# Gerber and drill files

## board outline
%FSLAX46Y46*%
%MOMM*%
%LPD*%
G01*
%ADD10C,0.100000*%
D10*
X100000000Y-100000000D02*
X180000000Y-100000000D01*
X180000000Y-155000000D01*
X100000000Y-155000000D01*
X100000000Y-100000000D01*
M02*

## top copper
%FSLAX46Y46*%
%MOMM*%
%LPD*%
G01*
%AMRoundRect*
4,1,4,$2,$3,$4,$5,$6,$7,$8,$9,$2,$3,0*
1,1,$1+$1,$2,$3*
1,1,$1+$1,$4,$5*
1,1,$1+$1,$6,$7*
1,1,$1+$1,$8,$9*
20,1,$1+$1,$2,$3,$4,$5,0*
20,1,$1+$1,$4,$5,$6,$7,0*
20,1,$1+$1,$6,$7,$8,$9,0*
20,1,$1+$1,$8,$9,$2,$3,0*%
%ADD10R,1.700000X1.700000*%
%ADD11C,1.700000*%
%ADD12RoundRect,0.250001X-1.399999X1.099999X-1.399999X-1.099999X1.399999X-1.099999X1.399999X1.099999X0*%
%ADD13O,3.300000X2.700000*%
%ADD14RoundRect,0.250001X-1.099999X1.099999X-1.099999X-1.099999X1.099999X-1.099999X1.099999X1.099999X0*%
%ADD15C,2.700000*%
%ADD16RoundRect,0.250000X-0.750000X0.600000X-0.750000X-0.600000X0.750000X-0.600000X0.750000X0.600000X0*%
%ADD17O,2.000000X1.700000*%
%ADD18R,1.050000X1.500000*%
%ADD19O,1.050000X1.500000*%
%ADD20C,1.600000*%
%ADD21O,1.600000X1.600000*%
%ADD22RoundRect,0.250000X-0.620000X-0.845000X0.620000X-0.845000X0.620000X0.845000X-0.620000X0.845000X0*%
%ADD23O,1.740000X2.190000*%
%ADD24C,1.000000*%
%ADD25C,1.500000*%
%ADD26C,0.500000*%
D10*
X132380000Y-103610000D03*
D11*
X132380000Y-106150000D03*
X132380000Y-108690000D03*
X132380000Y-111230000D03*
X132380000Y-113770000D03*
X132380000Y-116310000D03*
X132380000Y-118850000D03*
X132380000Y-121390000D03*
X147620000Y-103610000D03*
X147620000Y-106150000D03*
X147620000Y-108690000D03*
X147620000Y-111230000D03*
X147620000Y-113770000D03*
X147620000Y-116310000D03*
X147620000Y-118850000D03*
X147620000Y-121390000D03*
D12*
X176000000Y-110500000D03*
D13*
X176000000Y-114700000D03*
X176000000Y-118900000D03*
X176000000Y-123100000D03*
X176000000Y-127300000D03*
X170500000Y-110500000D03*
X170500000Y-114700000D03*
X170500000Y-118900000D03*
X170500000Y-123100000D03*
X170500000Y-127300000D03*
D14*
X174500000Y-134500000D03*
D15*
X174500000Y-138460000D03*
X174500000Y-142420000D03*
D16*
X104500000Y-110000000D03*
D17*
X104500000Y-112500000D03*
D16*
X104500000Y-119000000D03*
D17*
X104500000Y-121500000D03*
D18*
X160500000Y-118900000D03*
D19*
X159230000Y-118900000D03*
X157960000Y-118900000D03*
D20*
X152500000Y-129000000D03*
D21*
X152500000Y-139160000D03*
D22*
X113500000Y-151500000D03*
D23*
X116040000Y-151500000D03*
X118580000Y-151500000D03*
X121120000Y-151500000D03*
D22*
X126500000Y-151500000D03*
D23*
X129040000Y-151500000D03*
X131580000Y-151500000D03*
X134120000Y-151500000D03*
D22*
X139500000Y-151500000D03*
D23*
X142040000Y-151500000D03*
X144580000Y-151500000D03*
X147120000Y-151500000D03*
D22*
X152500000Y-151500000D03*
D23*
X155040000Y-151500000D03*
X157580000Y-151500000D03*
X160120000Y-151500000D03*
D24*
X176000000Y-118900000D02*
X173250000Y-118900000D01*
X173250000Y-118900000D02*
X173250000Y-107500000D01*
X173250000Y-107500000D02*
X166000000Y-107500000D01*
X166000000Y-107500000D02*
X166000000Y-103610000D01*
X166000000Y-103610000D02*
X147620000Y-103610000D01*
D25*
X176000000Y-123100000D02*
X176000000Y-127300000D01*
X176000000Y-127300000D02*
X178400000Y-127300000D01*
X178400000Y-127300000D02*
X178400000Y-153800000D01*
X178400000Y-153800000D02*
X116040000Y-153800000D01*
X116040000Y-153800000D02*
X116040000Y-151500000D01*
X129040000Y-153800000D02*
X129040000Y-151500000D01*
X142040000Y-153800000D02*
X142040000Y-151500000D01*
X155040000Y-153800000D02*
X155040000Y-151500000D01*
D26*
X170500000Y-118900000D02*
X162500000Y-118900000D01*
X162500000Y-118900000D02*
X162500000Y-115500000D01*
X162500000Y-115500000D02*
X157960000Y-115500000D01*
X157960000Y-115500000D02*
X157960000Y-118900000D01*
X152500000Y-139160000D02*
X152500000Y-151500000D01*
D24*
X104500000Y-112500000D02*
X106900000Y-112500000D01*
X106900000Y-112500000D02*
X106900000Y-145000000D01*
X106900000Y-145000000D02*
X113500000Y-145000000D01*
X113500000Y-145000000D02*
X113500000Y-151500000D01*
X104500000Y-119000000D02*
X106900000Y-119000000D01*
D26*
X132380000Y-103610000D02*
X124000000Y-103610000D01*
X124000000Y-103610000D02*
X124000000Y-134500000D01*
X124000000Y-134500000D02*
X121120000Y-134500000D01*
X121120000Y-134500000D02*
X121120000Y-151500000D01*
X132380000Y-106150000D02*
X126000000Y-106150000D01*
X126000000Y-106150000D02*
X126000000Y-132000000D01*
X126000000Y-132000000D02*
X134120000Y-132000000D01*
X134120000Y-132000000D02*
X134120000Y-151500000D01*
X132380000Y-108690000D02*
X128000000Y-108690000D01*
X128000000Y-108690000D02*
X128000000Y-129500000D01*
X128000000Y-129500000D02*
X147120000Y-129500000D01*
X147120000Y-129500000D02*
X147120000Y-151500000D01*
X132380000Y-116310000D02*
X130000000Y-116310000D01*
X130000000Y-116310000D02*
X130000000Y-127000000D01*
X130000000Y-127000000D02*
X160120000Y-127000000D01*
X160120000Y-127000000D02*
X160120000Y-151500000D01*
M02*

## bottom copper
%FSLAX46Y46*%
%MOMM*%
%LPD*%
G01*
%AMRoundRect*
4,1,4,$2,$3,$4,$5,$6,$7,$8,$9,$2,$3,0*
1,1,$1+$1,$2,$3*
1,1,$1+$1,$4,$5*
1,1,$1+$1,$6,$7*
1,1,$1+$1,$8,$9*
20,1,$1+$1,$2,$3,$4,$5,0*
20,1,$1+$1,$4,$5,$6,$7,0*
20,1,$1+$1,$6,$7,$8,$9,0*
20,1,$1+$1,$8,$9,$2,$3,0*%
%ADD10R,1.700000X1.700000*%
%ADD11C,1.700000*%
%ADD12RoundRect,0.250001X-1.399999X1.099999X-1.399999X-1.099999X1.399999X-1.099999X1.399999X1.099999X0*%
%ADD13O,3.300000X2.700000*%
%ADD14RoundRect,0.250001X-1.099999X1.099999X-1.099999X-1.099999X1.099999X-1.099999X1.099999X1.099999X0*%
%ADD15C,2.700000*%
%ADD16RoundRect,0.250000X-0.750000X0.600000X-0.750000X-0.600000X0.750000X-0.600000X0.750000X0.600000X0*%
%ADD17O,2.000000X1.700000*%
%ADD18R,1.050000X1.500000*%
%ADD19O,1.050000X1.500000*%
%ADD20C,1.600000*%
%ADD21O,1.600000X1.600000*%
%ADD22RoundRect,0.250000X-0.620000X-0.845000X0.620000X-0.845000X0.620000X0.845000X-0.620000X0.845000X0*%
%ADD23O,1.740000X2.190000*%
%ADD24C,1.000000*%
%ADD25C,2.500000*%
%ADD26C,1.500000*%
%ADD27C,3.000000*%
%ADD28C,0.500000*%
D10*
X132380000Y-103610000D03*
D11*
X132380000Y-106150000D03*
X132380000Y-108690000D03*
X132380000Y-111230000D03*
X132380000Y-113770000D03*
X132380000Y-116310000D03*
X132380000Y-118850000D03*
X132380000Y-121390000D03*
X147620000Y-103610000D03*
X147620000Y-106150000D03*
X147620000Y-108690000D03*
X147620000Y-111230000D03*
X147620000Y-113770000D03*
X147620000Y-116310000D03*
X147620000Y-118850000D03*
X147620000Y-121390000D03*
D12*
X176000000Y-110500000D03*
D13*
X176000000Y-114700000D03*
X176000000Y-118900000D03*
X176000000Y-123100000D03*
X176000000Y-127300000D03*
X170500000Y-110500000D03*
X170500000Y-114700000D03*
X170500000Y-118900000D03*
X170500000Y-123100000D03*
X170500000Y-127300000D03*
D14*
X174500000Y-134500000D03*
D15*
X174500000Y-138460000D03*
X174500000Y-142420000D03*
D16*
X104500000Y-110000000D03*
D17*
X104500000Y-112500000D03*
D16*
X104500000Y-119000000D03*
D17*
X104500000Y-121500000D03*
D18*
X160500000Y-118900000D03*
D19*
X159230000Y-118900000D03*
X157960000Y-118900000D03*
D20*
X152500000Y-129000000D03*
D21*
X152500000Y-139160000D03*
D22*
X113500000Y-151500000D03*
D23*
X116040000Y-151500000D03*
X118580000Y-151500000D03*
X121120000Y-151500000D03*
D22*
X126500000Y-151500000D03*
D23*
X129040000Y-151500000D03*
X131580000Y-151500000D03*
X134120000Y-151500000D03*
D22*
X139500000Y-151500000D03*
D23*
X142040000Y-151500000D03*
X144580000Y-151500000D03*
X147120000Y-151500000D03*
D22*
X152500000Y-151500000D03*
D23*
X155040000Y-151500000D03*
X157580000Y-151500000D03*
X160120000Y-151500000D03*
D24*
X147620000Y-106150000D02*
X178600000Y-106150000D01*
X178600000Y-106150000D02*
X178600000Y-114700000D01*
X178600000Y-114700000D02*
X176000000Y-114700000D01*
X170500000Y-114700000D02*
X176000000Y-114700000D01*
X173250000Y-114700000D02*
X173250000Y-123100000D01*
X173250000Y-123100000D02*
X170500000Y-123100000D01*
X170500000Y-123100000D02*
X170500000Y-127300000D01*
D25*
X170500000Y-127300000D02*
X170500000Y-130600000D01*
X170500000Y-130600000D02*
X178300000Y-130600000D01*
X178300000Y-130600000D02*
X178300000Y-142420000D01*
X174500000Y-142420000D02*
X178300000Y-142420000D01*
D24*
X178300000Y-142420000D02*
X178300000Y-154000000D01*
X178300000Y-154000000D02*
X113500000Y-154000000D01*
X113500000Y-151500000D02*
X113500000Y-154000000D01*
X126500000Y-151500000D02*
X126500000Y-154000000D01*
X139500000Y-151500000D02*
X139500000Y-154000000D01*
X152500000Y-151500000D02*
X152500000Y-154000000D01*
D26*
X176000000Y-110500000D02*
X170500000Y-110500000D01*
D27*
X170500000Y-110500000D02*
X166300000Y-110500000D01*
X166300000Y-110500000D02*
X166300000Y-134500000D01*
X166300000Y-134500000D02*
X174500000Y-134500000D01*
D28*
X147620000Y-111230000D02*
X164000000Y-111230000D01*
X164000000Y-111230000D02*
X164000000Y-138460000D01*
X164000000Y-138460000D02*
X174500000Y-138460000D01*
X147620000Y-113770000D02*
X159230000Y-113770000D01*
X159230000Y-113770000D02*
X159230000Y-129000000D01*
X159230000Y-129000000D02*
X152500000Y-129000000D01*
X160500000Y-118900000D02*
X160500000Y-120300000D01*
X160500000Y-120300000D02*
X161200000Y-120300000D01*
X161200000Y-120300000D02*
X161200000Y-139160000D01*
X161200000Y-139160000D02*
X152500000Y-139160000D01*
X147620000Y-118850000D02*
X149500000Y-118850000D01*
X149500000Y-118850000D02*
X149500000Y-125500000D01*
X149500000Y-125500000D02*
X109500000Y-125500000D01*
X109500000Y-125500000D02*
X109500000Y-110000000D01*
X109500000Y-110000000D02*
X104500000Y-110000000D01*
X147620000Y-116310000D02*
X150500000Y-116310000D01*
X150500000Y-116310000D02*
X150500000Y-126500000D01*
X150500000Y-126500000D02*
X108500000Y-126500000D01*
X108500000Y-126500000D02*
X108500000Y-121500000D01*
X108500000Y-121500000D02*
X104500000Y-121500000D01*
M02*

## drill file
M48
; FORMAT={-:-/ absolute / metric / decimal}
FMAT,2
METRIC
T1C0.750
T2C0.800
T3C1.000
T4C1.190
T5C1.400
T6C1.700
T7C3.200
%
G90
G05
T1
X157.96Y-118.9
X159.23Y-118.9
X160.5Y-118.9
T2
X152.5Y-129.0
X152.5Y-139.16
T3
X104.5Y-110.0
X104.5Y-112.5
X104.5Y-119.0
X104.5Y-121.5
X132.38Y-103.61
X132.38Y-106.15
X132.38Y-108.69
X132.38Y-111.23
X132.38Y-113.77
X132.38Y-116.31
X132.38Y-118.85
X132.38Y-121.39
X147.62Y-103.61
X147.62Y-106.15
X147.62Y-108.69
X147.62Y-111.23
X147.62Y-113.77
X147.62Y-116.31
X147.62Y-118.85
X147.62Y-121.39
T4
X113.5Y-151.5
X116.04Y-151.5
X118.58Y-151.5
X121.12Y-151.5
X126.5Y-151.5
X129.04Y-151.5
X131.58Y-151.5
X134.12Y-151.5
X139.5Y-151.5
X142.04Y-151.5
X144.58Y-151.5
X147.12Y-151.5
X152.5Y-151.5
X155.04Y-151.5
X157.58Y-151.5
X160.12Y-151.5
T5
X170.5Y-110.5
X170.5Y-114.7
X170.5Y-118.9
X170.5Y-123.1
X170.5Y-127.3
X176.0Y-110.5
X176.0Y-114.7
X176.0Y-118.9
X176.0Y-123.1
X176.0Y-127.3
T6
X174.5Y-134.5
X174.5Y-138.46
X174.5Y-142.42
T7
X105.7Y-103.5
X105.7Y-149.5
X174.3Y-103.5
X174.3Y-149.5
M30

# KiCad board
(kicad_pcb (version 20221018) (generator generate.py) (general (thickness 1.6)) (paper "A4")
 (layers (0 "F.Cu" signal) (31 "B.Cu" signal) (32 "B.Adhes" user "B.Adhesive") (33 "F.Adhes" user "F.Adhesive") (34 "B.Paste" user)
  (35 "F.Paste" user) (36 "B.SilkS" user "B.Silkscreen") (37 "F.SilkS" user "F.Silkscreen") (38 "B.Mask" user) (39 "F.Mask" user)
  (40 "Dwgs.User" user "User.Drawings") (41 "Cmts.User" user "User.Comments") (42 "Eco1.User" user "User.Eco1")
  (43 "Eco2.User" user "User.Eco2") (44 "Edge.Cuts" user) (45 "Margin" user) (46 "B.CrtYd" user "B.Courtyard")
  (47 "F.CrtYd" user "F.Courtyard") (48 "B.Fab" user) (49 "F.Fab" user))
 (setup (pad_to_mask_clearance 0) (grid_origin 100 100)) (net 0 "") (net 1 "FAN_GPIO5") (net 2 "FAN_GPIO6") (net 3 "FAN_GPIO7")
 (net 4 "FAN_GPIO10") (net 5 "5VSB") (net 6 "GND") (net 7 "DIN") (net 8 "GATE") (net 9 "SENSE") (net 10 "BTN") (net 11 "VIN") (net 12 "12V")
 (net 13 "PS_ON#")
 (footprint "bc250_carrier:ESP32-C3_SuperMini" (layer "F.Cu") (at 140 112.5 0)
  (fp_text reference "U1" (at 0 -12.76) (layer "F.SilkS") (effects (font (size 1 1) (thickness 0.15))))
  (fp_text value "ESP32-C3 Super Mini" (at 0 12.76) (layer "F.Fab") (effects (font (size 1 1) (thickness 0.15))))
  (pad "1" thru_hole rect (at -7.62 -8.89) (size 1.7 1.7) (drill 1) (layers "*.Cu" "*.Mask") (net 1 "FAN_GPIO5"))
  (pad "2" thru_hole circle (at -7.62 -6.35) (size 1.7 1.7) (drill 1) (layers "*.Cu" "*.Mask") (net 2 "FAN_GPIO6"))
  (pad "3" thru_hole circle (at -7.62 -3.81) (size 1.7 1.7) (drill 1) (layers "*.Cu" "*.Mask") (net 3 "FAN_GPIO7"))
  (pad "4" thru_hole circle (at -7.62 -1.27) (size 1.7 1.7) (drill 1) (layers "*.Cu" "*.Mask"))
  (pad "5" thru_hole circle (at -7.62 1.27) (size 1.7 1.7) (drill 1) (layers "*.Cu" "*.Mask"))
  (pad "6" thru_hole circle (at -7.62 3.81) (size 1.7 1.7) (drill 1) (layers "*.Cu" "*.Mask") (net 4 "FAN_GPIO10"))
  (pad "7" thru_hole circle (at -7.62 6.35) (size 1.7 1.7) (drill 1) (layers "*.Cu" "*.Mask"))
  (pad "8" thru_hole circle (at -7.62 8.89) (size 1.7 1.7) (drill 1) (layers "*.Cu" "*.Mask"))
  (pad "9" thru_hole circle (at 7.62 -8.89) (size 1.7 1.7) (drill 1) (layers "*.Cu" "*.Mask") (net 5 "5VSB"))
  (pad "10" thru_hole circle (at 7.62 -6.35) (size 1.7 1.7) (drill 1) (layers "*.Cu" "*.Mask") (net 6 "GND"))
  (pad "11" thru_hole circle (at 7.62 -3.81) (size 1.7 1.7) (drill 1) (layers "*.Cu" "*.Mask"))
  (pad "12" thru_hole circle (at 7.62 -1.27) (size 1.7 1.7) (drill 1) (layers "*.Cu" "*.Mask") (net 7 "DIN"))
  (pad "13" thru_hole circle (at 7.62 1.27) (size 1.7 1.7) (drill 1) (layers "*.Cu" "*.Mask") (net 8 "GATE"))
  (pad "14" thru_hole circle (at 7.62 3.81) (size 1.7 1.7) (drill 1) (layers "*.Cu" "*.Mask") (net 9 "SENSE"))
  (pad "15" thru_hole circle (at 7.62 6.35) (size 1.7 1.7) (drill 1) (layers "*.Cu" "*.Mask") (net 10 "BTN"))
  (pad "16" thru_hole circle (at 7.62 8.89) (size 1.7 1.7) (drill 1) (layers "*.Cu" "*.Mask")))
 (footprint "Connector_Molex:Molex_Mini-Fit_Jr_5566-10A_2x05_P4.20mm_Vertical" (layer "F.Cu") (at 176 110.5 270)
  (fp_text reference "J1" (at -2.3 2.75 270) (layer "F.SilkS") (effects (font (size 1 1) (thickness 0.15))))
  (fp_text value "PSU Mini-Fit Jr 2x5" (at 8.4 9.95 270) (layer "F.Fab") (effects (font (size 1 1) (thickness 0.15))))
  (pad "1" thru_hole roundrect (at 0 0 270) (size 2.7 3.3) (drill 1.4) (layers *.Cu *.Mask) (roundrect_rratio 0.092593) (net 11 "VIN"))
  (pad "2" thru_hole oval (at 4.2 0 270) (size 2.7 3.3) (drill 1.4) (layers *.Cu *.Mask) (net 6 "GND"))
  (pad "3" thru_hole oval (at 8.4 0 270) (size 2.7 3.3) (drill 1.4) (layers *.Cu *.Mask) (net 5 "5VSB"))
  (pad "4" thru_hole oval (at 12.6 0 270) (size 2.7 3.3) (drill 1.4) (layers *.Cu *.Mask) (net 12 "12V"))
  (pad "5" thru_hole oval (at 16.8 0 270) (size 2.7 3.3) (drill 1.4) (layers *.Cu *.Mask) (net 12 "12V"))
  (pad "6" thru_hole oval (at 0 5.5 270) (size 2.7 3.3) (drill 1.4) (layers *.Cu *.Mask) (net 11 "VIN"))
  (pad "7" thru_hole oval (at 4.2 5.5 270) (size 2.7 3.3) (drill 1.4) (layers *.Cu *.Mask) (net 6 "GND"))
  (pad "8" thru_hole oval (at 8.4 5.5 270) (size 2.7 3.3) (drill 1.4) (layers *.Cu *.Mask) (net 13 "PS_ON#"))
  (pad "9" thru_hole oval (at 12.6 5.5 270) (size 2.7 3.3) (drill 1.4) (layers *.Cu *.Mask) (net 6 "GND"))
  (pad "10" thru_hole oval (at 16.8 5.5 270) (size 2.7 3.3) (drill 1.4) (layers *.Cu *.Mask) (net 6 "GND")))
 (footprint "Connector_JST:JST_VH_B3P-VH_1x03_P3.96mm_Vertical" (layer "F.Cu") (at 174.5 134.5 270)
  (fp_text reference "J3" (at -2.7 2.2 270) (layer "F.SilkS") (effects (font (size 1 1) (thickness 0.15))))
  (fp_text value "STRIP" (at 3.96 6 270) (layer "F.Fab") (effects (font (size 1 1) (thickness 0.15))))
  (pad "1" thru_hole roundrect (at 0 0 270) (size 2.7 2.7) (drill 1.7) (layers *.Cu *.Mask) (roundrect_rratio 0.092593) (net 11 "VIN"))
  (pad "2" thru_hole circle (at 3.96 0 270) (size 2.7 2.7) (drill 1.7) (layers *.Cu *.Mask) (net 7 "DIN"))
  (pad "3" thru_hole circle (at 7.92 0 270) (size 2.7 2.7) (drill 1.7) (layers *.Cu *.Mask) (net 6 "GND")))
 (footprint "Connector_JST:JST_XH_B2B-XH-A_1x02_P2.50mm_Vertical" (layer "F.Cu") (at 104.5 110 270)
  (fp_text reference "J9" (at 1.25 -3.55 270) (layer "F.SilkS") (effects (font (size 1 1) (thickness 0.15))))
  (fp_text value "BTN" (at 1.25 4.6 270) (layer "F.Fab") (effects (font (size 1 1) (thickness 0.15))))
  (pad "1" thru_hole roundrect (at 0 0 270) (size 1.7 2) (drill 1) (layers *.Cu *.Mask) (roundrect_rratio 0.147059) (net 10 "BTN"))
  (pad "2" thru_hole oval (at 2.5 0 270) (size 1.7 2) (drill 1) (layers *.Cu *.Mask) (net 6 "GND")))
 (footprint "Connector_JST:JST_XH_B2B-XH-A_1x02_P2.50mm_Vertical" (layer "F.Cu") (at 104.5 119 270)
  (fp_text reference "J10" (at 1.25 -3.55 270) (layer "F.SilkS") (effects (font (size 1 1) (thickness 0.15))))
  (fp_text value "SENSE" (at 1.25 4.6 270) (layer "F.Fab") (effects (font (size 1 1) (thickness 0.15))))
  (pad "1" thru_hole roundrect (at 0 0 270) (size 1.7 2) (drill 1) (layers *.Cu *.Mask) (roundrect_rratio 0.147059) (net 6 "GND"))
  (pad "2" thru_hole oval (at 2.5 0 270) (size 1.7 2) (drill 1) (layers *.Cu *.Mask) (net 9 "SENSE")))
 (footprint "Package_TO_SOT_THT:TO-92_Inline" (layer "F.Cu") (at 160.5 118.9 180)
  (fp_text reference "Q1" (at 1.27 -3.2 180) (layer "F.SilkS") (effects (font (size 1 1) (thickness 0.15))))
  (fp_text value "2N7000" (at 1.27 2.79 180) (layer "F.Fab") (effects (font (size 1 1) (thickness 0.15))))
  (pad "1" thru_hole rect (at 0 0 180) (size 1.05 1.5) (drill 0.75) (layers *.Cu *.Mask) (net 6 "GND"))
  (pad "2" thru_hole oval (at 1.27 0 180) (size 1.05 1.5) (drill 0.75) (layers *.Cu *.Mask) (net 8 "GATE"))
  (pad "3" thru_hole oval (at 2.54 0 180) (size 1.05 1.5) (drill 0.75) (layers *.Cu *.Mask) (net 13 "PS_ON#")))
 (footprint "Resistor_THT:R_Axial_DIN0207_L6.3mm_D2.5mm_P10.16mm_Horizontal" (layer "F.Cu") (at 152.5 129 270)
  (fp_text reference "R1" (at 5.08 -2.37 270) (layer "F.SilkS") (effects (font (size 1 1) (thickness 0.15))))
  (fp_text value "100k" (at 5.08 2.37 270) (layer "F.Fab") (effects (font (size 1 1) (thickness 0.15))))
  (pad "1" thru_hole circle (at 0 0 270) (size 1.6 1.6) (drill 0.8) (layers *.Cu *.Mask) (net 8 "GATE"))
  (pad "2" thru_hole oval (at 10.16 0 270) (size 1.6 1.6) (drill 0.8) (layers *.Cu *.Mask) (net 6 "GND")))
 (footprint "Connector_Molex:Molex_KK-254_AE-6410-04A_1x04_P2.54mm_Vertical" (layer "F.Cu") (at 113.5 151.5 0)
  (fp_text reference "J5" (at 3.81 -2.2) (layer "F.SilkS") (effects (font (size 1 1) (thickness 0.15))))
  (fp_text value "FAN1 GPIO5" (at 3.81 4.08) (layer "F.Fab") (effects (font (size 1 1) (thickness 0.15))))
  (pad "1" thru_hole roundrect (at 0 0) (size 1.74 2.19) (drill 1.19) (layers *.Cu *.Mask) (roundrect_rratio 0.143678) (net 6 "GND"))
  (pad "2" thru_hole oval (at 2.54 0) (size 1.74 2.19) (drill 1.19) (layers *.Cu *.Mask) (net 12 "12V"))
  (pad "3" thru_hole oval (at 5.08 0) (size 1.74 2.19) (drill 1.19) (layers *.Cu *.Mask))
  (pad "4" thru_hole oval (at 7.62 0) (size 1.74 2.19) (drill 1.19) (layers *.Cu *.Mask) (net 1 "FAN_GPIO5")))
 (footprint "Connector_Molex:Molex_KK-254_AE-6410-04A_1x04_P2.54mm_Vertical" (layer "F.Cu") (at 126.5 151.5 0)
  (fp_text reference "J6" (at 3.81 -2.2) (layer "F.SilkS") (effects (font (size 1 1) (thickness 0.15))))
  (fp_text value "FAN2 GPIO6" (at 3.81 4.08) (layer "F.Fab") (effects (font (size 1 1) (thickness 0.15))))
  (pad "1" thru_hole roundrect (at 0 0) (size 1.74 2.19) (drill 1.19) (layers *.Cu *.Mask) (roundrect_rratio 0.143678) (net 6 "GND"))
  (pad "2" thru_hole oval (at 2.54 0) (size 1.74 2.19) (drill 1.19) (layers *.Cu *.Mask) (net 12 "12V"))
  (pad "3" thru_hole oval (at 5.08 0) (size 1.74 2.19) (drill 1.19) (layers *.Cu *.Mask))
  (pad "4" thru_hole oval (at 7.62 0) (size 1.74 2.19) (drill 1.19) (layers *.Cu *.Mask) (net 2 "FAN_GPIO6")))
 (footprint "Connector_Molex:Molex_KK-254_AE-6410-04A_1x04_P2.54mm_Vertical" (layer "F.Cu") (at 139.5 151.5 0)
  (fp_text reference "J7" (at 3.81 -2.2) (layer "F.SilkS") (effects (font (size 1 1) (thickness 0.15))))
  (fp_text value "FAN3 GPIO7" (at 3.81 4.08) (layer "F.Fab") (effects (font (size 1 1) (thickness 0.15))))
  (pad "1" thru_hole roundrect (at 0 0) (size 1.74 2.19) (drill 1.19) (layers *.Cu *.Mask) (roundrect_rratio 0.143678) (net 6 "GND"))
  (pad "2" thru_hole oval (at 2.54 0) (size 1.74 2.19) (drill 1.19) (layers *.Cu *.Mask) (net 12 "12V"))
  (pad "3" thru_hole oval (at 5.08 0) (size 1.74 2.19) (drill 1.19) (layers *.Cu *.Mask))
  (pad "4" thru_hole oval (at 7.62 0) (size 1.74 2.19) (drill 1.19) (layers *.Cu *.Mask) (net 3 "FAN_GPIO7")))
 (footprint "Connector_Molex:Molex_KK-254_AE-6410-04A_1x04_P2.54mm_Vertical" (layer "F.Cu") (at 152.5 151.5 0)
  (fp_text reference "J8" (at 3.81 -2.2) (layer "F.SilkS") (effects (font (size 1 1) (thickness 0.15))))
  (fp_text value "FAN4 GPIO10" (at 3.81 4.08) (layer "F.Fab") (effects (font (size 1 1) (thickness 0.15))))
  (pad "1" thru_hole roundrect (at 0 0) (size 1.74 2.19) (drill 1.19) (layers *.Cu *.Mask) (roundrect_rratio 0.143678) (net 6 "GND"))
  (pad "2" thru_hole oval (at 2.54 0) (size 1.74 2.19) (drill 1.19) (layers *.Cu *.Mask) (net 12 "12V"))
  (pad "3" thru_hole oval (at 5.08 0) (size 1.74 2.19) (drill 1.19) (layers *.Cu *.Mask))
  (pad "4" thru_hole oval (at 7.62 0) (size 1.74 2.19) (drill 1.19) (layers *.Cu *.Mask) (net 4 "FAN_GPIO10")))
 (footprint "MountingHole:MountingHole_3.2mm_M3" (layer "F.Cu") (at 105.7 103.5 0)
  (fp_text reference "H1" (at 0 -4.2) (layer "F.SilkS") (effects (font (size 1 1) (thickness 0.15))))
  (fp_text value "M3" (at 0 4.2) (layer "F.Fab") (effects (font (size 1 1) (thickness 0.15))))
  (pad "" np_thru_hole circle (at 0 0) (size 3.2 3.2) (drill 3.2) (layers *.Cu *.Mask)))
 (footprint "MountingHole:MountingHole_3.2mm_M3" (layer "F.Cu") (at 174.3 103.5 0)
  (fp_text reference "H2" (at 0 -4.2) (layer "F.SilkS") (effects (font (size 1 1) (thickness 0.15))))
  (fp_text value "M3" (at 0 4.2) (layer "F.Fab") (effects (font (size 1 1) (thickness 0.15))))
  (pad "" np_thru_hole circle (at 0 0) (size 3.2 3.2) (drill 3.2) (layers *.Cu *.Mask)))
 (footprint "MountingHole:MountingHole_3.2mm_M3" (layer "F.Cu") (at 105.7 149.5 0)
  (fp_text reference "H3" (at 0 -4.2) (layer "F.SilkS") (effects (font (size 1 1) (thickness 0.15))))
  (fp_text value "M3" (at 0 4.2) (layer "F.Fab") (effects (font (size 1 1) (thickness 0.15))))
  (pad "" np_thru_hole circle (at 0 0) (size 3.2 3.2) (drill 3.2) (layers *.Cu *.Mask)))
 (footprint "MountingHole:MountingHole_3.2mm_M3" (layer "F.Cu") (at 174.3 149.5 0)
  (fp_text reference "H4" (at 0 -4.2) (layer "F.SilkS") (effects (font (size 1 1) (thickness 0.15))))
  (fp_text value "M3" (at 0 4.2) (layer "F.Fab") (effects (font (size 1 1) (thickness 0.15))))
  (pad "" np_thru_hole circle (at 0 0) (size 3.2 3.2) (drill 3.2) (layers *.Cu *.Mask)))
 (gr_rect (start 100 100) (end 180 155) (stroke (width 0.1) (type default)) (fill none) (layer "Edge.Cuts"))
 (segment (start 176 118.9) (end 173.25 118.9) (width 1) (layer "F.Cu") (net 5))
 (segment (start 173.25 118.9) (end 173.25 107.5) (width 1) (layer "F.Cu") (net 5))
 (segment (start 173.25 107.5) (end 166 107.5) (width 1) (layer "F.Cu") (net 5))
 (segment (start 166 107.5) (end 166 103.61) (width 1) (layer "F.Cu") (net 5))
 (segment (start 166 103.61) (end 147.62 103.61) (width 1) (layer "F.Cu") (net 5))
 (segment (start 147.62 106.15) (end 178.6 106.15) (width 1) (layer "B.Cu") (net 6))
 (segment (start 178.6 106.15) (end 178.6 114.7) (width 1) (layer "B.Cu") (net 6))
 (segment (start 178.6 114.7) (end 176 114.7) (width 1) (layer "B.Cu") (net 6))
 (segment (start 170.5 114.7) (end 176 114.7) (width 1) (layer "B.Cu") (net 6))
 (segment (start 173.25 114.7) (end 173.25 123.1) (width 1) (layer "B.Cu") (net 6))
 (segment (start 173.25 123.1) (end 170.5 123.1) (width 1) (layer "B.Cu") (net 6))
 (segment (start 170.5 123.1) (end 170.5 127.3) (width 1) (layer "B.Cu") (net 6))
 (segment (start 170.5 127.3) (end 170.5 130.6) (width 2.5) (layer "B.Cu") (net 6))
 (segment (start 170.5 130.6) (end 178.3 130.6) (width 2.5) (layer "B.Cu") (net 6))
 (segment (start 178.3 130.6) (end 178.3 142.42) (width 2.5) (layer "B.Cu") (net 6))
 (segment (start 174.5 142.42) (end 178.3 142.42) (width 2.5) (layer "B.Cu") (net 6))
 (segment (start 178.3 142.42) (end 178.3 154) (width 1) (layer "B.Cu") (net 6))
 (segment (start 178.3 154) (end 113.5 154) (width 1) (layer "B.Cu") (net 6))
 (segment (start 176 123.1) (end 176 127.3) (width 1.5) (layer "F.Cu") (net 12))
 (segment (start 176 127.3) (end 178.4 127.3) (width 1.5) (layer "F.Cu") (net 12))
 (segment (start 178.4 127.3) (end 178.4 153.8) (width 1.5) (layer "F.Cu") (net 12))
 (segment (start 178.4 153.8) (end 116.04 153.8) (width 1.5) (layer "F.Cu") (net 12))
 (segment (start 116.04 153.8) (end 116.04 151.5) (width 1.5) (layer "F.Cu") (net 12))
 (segment (start 113.5 151.5) (end 113.5 154) (width 1) (layer "B.Cu") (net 6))
 (segment (start 129.04 153.8) (end 129.04 151.5) (width 1.5) (layer "F.Cu") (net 12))
 (segment (start 126.5 151.5) (end 126.5 154) (width 1) (layer "B.Cu") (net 6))
 (segment (start 142.04 153.8) (end 142.04 151.5) (width 1.5) (layer "F.Cu") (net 12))
 (segment (start 139.5 151.5) (end 139.5 154) (width 1) (layer "B.Cu") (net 6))
 (segment (start 155.04 153.8) (end 155.04 151.5) (width 1.5) (layer "F.Cu") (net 12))
 (segment (start 152.5 151.5) (end 152.5 154) (width 1) (layer "B.Cu") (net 6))
 (segment (start 176 110.5) (end 170.5 110.5) (width 1.5) (layer "B.Cu") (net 11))
 (segment (start 170.5 110.5) (end 166.3 110.5) (width 3) (layer "B.Cu") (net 11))
 (segment (start 166.3 110.5) (end 166.3 134.5) (width 3) (layer "B.Cu") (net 11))
 (segment (start 166.3 134.5) (end 174.5 134.5) (width 3) (layer "B.Cu") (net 11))
 (segment (start 147.62 111.23) (end 164 111.23) (width 0.5) (layer "B.Cu") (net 7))
 (segment (start 164 111.23) (end 164 138.46) (width 0.5) (layer "B.Cu") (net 7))
 (segment (start 164 138.46) (end 174.5 138.46) (width 0.5) (layer "B.Cu") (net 7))
 (segment (start 170.5 118.9) (end 162.5 118.9) (width 0.5) (layer "F.Cu") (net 13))
 (segment (start 162.5 118.9) (end 162.5 115.5) (width 0.5) (layer "F.Cu") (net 13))
 (segment (start 162.5 115.5) (end 157.96 115.5) (width 0.5) (layer "F.Cu") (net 13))
 (segment (start 157.96 115.5) (end 157.96 118.9) (width 0.5) (layer "F.Cu") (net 13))
 (segment (start 147.62 113.77) (end 159.23 113.77) (width 0.5) (layer "B.Cu") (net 8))
 (segment (start 159.23 113.77) (end 159.23 129) (width 0.5) (layer "B.Cu") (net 8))
 (segment (start 159.23 129) (end 152.5 129) (width 0.5) (layer "B.Cu") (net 8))
 (segment (start 160.5 118.9) (end 160.5 120.3) (width 0.5) (layer "B.Cu") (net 6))
 (segment (start 160.5 120.3) (end 161.2 120.3) (width 0.5) (layer "B.Cu") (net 6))
 (segment (start 161.2 120.3) (end 161.2 139.16) (width 0.5) (layer "B.Cu") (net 6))
 (segment (start 161.2 139.16) (end 152.5 139.16) (width 0.5) (layer "B.Cu") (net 6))
 (segment (start 152.5 139.16) (end 152.5 151.5) (width 0.5) (layer "F.Cu") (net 6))
 (segment (start 147.62 118.85) (end 149.5 118.85) (width 0.5) (layer "B.Cu") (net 10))
 (segment (start 149.5 118.85) (end 149.5 125.5) (width 0.5) (layer "B.Cu") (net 10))
 (segment (start 149.5 125.5) (end 109.5 125.5) (width 0.5) (layer "B.Cu") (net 10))
 (segment (start 109.5 125.5) (end 109.5 110) (width 0.5) (layer "B.Cu") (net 10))
 (segment (start 109.5 110) (end 104.5 110) (width 0.5) (layer "B.Cu") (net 10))
 (segment (start 147.62 116.31) (end 150.5 116.31) (width 0.5) (layer "B.Cu") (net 9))
 (segment (start 150.5 116.31) (end 150.5 126.5) (width 0.5) (layer "B.Cu") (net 9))
 (segment (start 150.5 126.5) (end 108.5 126.5) (width 0.5) (layer "B.Cu") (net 9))
 (segment (start 108.5 126.5) (end 108.5 121.5) (width 0.5) (layer "B.Cu") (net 9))
 (segment (start 108.5 121.5) (end 104.5 121.5) (width 0.5) (layer "B.Cu") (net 9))
 (segment (start 104.5 112.5) (end 106.9 112.5) (width 1) (layer "F.Cu") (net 6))
 (segment (start 106.9 112.5) (end 106.9 145) (width 1) (layer "F.Cu") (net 6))
 (segment (start 106.9 145) (end 113.5 145) (width 1) (layer "F.Cu") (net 6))
 (segment (start 113.5 145) (end 113.5 151.5) (width 1) (layer "F.Cu") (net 6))
 (segment (start 104.5 119) (end 106.9 119) (width 1) (layer "F.Cu") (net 6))
 (segment (start 132.38 103.61) (end 124 103.61) (width 0.5) (layer "F.Cu") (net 1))
 (segment (start 124 103.61) (end 124 134.5) (width 0.5) (layer "F.Cu") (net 1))
 (segment (start 124 134.5) (end 121.12 134.5) (width 0.5) (layer "F.Cu") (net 1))
 (segment (start 121.12 134.5) (end 121.12 151.5) (width 0.5) (layer "F.Cu") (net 1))
 (segment (start 132.38 106.15) (end 126 106.15) (width 0.5) (layer "F.Cu") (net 2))
 (segment (start 126 106.15) (end 126 132) (width 0.5) (layer "F.Cu") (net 2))
 (segment (start 126 132) (end 134.12 132) (width 0.5) (layer "F.Cu") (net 2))
 (segment (start 134.12 132) (end 134.12 151.5) (width 0.5) (layer "F.Cu") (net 2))
 (segment (start 132.38 108.69) (end 128 108.69) (width 0.5) (layer "F.Cu") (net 3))
 (segment (start 128 108.69) (end 128 129.5) (width 0.5) (layer "F.Cu") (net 3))
 (segment (start 128 129.5) (end 147.12 129.5) (width 0.5) (layer "F.Cu") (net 3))
 (segment (start 147.12 129.5) (end 147.12 151.5) (width 0.5) (layer "F.Cu") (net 3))
 (segment (start 132.38 116.31) (end 130 116.31) (width 0.5) (layer "F.Cu") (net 4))
 (segment (start 130 116.31) (end 130 127) (width 0.5) (layer "F.Cu") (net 4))
 (segment (start 130 127) (end 160.12 127) (width 0.5) (layer "F.Cu") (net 4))
 (segment (start 160.12 127) (end 160.12 151.5) (width 0.5) (layer "F.Cu") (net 4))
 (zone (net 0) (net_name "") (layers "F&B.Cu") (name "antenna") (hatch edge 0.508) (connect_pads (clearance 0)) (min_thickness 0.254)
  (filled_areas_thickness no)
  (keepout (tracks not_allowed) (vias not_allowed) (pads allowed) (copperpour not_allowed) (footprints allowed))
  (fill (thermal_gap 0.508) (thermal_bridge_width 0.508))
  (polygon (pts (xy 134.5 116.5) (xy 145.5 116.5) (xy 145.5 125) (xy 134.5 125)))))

